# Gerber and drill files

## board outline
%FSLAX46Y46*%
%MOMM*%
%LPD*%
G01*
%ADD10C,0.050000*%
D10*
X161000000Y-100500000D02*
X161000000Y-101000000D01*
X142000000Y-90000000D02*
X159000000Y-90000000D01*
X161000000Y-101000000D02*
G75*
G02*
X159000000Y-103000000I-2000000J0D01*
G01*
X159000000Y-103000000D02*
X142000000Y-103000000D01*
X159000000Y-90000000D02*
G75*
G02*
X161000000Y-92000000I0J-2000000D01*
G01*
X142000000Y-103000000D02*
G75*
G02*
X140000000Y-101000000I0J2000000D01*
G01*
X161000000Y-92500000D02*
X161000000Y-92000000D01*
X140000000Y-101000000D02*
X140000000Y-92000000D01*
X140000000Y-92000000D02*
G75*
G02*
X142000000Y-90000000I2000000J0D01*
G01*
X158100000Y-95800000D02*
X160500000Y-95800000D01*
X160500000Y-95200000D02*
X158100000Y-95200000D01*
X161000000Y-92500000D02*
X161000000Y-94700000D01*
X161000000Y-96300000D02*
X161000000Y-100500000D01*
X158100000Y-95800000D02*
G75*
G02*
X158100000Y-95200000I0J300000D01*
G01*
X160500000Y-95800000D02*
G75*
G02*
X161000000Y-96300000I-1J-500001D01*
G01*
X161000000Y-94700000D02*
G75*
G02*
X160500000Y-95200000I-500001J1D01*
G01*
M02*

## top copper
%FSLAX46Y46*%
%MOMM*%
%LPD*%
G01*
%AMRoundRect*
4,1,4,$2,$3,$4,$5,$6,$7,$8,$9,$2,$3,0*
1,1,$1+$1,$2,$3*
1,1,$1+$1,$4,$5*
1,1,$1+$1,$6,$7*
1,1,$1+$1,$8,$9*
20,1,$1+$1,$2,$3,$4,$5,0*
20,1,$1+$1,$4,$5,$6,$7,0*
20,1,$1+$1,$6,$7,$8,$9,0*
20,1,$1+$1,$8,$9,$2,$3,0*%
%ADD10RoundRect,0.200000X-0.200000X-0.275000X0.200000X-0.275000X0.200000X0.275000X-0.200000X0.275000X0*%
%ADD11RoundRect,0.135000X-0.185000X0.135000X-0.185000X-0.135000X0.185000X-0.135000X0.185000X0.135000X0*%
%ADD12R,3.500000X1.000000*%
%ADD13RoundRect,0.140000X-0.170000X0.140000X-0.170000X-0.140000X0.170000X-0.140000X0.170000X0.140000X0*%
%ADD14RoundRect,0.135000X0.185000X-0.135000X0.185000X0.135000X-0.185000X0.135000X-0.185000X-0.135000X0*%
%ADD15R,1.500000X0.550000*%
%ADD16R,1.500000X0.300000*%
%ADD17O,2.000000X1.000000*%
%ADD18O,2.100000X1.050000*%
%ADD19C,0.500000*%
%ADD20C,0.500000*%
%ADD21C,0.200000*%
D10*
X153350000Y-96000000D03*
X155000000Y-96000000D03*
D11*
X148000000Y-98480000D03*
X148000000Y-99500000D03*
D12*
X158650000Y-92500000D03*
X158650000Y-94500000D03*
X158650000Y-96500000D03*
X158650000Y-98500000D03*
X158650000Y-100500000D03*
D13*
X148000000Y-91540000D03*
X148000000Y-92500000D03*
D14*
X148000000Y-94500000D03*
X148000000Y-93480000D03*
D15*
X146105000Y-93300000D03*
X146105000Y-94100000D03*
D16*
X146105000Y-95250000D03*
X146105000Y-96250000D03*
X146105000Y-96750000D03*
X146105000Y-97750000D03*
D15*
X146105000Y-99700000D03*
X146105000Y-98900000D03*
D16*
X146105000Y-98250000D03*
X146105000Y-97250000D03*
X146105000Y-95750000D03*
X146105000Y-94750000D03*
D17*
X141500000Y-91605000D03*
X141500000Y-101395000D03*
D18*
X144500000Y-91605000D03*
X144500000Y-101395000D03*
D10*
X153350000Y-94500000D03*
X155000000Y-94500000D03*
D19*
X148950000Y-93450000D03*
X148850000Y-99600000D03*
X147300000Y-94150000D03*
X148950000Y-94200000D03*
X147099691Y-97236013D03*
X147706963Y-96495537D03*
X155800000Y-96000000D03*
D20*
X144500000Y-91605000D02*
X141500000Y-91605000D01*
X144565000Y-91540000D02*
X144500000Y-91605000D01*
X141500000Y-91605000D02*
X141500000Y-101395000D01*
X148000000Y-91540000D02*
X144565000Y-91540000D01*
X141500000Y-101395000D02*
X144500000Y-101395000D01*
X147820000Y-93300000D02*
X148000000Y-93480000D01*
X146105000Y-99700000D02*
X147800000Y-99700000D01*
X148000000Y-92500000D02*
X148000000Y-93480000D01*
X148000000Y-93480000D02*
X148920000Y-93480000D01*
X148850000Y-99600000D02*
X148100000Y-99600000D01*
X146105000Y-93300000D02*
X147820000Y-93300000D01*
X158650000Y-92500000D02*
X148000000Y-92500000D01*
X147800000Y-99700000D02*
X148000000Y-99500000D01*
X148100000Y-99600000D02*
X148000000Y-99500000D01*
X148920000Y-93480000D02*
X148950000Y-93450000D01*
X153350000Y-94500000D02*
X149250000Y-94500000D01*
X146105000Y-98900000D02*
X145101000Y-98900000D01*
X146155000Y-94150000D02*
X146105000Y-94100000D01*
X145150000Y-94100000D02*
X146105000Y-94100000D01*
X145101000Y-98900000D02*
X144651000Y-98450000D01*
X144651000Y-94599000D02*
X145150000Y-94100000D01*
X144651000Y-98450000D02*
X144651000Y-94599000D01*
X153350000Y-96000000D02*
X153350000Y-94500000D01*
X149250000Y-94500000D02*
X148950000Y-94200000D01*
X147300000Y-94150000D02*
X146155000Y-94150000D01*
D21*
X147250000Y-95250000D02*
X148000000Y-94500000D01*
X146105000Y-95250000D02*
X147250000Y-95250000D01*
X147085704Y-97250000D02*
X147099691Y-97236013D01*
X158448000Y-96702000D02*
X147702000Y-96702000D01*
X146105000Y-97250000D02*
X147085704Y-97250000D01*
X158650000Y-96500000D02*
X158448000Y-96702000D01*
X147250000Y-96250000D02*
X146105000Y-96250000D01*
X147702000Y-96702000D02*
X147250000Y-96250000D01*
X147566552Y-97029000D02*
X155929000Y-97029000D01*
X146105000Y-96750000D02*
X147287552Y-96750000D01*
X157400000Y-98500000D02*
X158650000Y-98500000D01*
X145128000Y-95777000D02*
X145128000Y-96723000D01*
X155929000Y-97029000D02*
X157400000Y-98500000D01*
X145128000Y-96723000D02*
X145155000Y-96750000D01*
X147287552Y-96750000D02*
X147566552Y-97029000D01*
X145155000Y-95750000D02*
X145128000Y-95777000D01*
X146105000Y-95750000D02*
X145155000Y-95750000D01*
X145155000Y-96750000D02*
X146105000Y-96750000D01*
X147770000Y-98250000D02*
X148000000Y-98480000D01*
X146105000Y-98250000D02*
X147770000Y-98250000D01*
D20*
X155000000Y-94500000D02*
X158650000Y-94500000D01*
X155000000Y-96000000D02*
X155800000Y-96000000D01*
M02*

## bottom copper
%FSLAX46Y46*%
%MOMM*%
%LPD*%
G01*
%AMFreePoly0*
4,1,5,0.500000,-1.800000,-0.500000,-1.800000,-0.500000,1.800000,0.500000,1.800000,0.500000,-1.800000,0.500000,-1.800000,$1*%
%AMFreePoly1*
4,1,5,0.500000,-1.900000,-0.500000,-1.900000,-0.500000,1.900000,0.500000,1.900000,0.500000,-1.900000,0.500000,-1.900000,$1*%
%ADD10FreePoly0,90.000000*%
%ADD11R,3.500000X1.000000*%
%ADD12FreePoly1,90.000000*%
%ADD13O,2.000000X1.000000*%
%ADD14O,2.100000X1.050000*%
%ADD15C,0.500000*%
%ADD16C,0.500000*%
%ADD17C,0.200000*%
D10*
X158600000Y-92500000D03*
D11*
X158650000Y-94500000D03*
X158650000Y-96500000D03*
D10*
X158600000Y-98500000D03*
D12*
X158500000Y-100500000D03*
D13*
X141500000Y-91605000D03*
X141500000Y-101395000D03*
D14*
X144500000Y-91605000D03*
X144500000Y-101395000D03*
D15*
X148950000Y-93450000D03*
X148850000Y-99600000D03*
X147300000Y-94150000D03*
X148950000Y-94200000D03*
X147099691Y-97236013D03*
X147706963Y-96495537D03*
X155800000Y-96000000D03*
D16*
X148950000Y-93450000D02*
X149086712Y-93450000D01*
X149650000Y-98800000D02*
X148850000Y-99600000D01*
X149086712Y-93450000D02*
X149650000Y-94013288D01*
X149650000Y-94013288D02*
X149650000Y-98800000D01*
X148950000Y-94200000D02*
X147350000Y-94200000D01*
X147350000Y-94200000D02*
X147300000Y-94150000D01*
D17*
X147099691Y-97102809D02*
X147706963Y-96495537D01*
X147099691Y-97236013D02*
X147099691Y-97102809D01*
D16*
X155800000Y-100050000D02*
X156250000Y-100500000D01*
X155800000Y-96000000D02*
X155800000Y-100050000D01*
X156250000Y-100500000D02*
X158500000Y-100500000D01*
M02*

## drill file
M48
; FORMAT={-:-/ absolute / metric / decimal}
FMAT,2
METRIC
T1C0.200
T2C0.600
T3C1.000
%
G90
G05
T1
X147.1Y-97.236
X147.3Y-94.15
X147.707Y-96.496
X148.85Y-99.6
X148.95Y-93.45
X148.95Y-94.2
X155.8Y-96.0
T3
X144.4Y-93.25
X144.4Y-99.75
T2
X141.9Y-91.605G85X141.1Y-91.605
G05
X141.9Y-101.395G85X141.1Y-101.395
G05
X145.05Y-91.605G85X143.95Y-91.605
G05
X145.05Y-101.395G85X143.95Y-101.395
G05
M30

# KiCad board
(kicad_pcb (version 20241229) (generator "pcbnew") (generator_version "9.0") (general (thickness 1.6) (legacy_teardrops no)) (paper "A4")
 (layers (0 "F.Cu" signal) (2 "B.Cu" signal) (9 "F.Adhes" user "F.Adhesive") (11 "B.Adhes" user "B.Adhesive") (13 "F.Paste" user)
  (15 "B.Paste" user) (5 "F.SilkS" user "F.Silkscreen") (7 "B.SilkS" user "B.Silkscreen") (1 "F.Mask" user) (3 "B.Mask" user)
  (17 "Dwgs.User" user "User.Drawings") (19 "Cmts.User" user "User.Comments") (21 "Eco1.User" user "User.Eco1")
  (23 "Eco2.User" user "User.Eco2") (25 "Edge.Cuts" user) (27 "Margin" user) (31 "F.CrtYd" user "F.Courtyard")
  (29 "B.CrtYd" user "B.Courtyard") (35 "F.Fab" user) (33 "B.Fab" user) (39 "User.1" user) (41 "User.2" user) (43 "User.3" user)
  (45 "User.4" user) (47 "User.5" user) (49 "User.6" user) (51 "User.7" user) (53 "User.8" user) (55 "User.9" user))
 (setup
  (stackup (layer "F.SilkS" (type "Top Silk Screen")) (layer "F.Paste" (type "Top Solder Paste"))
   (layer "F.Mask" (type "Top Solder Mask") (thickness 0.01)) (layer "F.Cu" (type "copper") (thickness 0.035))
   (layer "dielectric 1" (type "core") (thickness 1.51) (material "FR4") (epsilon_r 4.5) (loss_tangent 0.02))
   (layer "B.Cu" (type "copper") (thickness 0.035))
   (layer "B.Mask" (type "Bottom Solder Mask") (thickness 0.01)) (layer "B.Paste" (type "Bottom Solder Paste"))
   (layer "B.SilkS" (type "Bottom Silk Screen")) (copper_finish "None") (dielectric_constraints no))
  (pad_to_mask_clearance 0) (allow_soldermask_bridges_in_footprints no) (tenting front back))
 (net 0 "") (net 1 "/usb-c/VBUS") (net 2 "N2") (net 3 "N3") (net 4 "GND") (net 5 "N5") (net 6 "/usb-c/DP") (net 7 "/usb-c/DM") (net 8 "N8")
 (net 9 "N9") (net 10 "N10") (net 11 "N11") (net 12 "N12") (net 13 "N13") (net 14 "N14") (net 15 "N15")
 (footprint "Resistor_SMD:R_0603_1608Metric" (layer "F.Cu") (at 154.175 96)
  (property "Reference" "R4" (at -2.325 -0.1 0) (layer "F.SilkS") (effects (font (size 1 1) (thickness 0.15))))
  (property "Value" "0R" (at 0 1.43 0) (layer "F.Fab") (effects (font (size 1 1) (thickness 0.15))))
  (pad "1" smd roundrect (at -0.825 0) (size 0.8 0.95) (layers "F.Cu" "F.Mask" "F.Paste") (roundrect_rratio 0.25) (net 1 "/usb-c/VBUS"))
  (pad "2" smd roundrect (at 0.825 0) (size 0.8 0.95) (layers "F.Cu" "F.Mask" "F.Paste") (roundrect_rratio 0.25) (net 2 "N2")))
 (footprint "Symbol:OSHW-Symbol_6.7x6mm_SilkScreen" (layer "F.Cu") (at 152 99.5)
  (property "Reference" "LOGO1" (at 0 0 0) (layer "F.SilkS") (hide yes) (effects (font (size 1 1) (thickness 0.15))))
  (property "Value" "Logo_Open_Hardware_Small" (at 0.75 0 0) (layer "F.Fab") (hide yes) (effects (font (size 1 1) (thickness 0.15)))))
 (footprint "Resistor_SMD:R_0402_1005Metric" (layer "F.Cu") (at 148 98.99 -90)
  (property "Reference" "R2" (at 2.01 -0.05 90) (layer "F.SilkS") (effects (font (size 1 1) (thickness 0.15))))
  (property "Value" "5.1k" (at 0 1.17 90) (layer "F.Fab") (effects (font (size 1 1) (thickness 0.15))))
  (pad "1" smd roundrect (at -0.51 0 270) (size 0.54 0.64) (layers "F.Cu" "F.Mask" "F.Paste") (roundrect_rratio 0.25) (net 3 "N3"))
  (pad "2" smd roundrect (at 0.51 0 270) (size 0.54 0.64) (layers "F.Cu" "F.Mask" "F.Paste") (roundrect_rratio 0.25) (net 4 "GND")))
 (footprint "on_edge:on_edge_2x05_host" (layer "F.Cu") (at 161 96.5 -90)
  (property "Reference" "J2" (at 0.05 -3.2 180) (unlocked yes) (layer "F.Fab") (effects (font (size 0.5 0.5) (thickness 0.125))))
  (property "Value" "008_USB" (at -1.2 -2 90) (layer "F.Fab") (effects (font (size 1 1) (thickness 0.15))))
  (fp_line (start -0.7 2.9) (end -0.7 0.5) (stroke (width 0.05) (type solid)) (layer "Edge.Cuts"))
  (fp_line (start -1.3 0.5) (end -1.3 2.9) (stroke (width 0.05) (type solid)) (layer "Edge.Cuts"))
  (fp_line (start -4 0) (end -1.8 0) (stroke (width 0.05) (type solid)) (layer "Edge.Cuts"))
  (fp_line (start -0.2 0) (end 4 0) (stroke (width 0.05) (type solid)) (layer "Edge.Cuts"))
  (fp_arc (start -0.7 2.9) (mid -1 3.2) (end -1.3 2.9) (stroke (width 0.05) (type solid)) (layer "Edge.Cuts"))
  (fp_arc (start -0.7 0.5) (mid -0.553553 0.146447) (end -0.2 0) (stroke (width 0.05) (type solid)) (layer "Edge.Cuts"))
  (fp_arc (start -1.8 0) (mid -1.446447 0.146447) (end -1.3 0.5) (stroke (width 0.05) (type solid)) (layer "Edge.Cuts"))
  (pad "1" smd rect (at -4 2.35 270) (size 1 3.5) (layers "F.Cu" "F.Mask") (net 4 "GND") (zone_connect 0))
  (pad "2" smd rect (at -2 2.35 270) (size 1 3.5) (layers "F.Cu" "F.Mask") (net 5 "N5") (zone_connect 0))
  (pad "3" smd rect (at 0 2.35 270) (size 1 3.5) (layers "F.Cu" "F.Mask") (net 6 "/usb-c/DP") (zone_connect 0))
  (pad "4" smd rect (at 2 2.35 270) (size 1 3.5) (layers "F.Cu" "F.Mask") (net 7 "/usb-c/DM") (zone_connect 0))
  (pad "5" smd rect (at 4 2.35 270) (size 1 3.5) (layers "F.Cu" "F.Mask") (zone_connect 0))
  (pad "6" smd custom (at -4 2.4 90) (size 1 3.6) (layers "B.Cu" "B.Mask") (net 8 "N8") (zone_connect 0)
   (options (clearance outline) (anchor rect)) (primitives))
  (pad "7" smd rect (at -2 2.35 90) (size 1 3.5) (layers "B.Cu" "B.Mask") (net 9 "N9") (zone_connect 0))
  (pad "8" smd rect (at 0 2.35 90) (size 1 3.5) (layers "B.Cu" "B.Mask") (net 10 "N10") (zone_connect 0))
  (pad "9" smd custom (at 2 2.4 90) (size 1 3.6) (layers "B.Cu" "B.Mask") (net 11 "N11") (zone_connect 0)
   (options (clearance outline) (anchor rect)) (primitives))
  (pad "10" smd custom (at 4 2.5 90) (size 1 3.8) (layers "B.Cu" "B.Mask") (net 2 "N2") (zone_connect 0)
   (options (clearance outline) (anchor rect)) (primitives))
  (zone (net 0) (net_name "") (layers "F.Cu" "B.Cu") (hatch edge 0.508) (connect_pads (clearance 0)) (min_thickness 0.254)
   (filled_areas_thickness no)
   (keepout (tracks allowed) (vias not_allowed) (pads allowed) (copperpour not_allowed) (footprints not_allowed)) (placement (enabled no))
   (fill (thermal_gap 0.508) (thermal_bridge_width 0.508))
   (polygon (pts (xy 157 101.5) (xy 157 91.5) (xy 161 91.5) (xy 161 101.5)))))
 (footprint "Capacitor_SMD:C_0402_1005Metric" (layer "F.Cu") (at 148 92.02 -90)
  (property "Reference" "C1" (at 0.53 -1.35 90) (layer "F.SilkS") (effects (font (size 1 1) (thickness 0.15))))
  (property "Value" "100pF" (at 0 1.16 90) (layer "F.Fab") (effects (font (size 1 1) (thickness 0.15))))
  (pad "1" smd roundrect (at -0.48 0 270) (size 0.56 0.62) (layers "F.Cu" "F.Mask" "F.Paste") (roundrect_rratio 0.25) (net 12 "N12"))
  (pad "2" smd roundrect (at 0.48 0 270) (size 0.56 0.62) (layers "F.Cu" "F.Mask" "F.Paste") (roundrect_rratio 0.25) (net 4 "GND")))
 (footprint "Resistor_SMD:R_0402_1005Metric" (layer "F.Cu") (at 148 93.99 90)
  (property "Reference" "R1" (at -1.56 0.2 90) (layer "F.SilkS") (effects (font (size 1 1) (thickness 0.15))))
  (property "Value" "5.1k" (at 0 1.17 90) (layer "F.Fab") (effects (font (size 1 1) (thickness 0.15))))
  (pad "1" smd roundrect (at -0.51 0 90) (size 0.54 0.64) (layers "F.Cu" "F.Mask" "F.Paste") (roundrect_rratio 0.25) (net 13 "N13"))
  (pad "2" smd roundrect (at 0.51 0 90) (size 0.54 0.64) (layers "F.Cu" "F.Mask" "F.Paste") (roundrect_rratio 0.25) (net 4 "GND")))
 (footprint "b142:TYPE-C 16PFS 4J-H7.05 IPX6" (layer "F.Cu") (at 143 96.5 -90)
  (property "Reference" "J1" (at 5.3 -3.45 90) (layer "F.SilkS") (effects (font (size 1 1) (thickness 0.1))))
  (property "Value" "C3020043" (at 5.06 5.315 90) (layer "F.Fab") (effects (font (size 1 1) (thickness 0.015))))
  (pad "" np_thru_hole circle (at -3.25 -1.4 270) (size 1 1) (drill 1) (layers "*.Cu" "*.Mask"))
  (pad "" np_thru_hole circle (at 3.25 -1.4 270) (size 1 1) (drill 1) (layers "*.Cu" "*.Mask"))
  (pad "A1/B12" smd rect (at -3.2 -3.105 270) (size 0.55 1.5) (layers "F.Cu" "F.Mask" "F.Paste") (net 4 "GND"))
  (pad "A4/B9" smd rect (at -2.4 -3.105 270) (size 0.55 1.5) (layers "F.Cu" "F.Mask" "F.Paste") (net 1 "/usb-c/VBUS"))
  (pad "A5" smd rect (at -1.25 -3.105 270) (size 0.3 1.5) (layers "F.Cu" "F.Mask" "F.Paste") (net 13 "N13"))
  (pad "A6" smd rect (at -0.25 -3.105 270) (size 0.3 1.5) (layers "F.Cu" "F.Mask" "F.Paste") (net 6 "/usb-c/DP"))
  (pad "A7" smd rect (at 0.25 -3.105 270) (size 0.3 1.5) (layers "F.Cu" "F.Mask" "F.Paste") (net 7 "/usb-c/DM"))
  (pad "A8" smd rect (at 1.25 -3.105 270) (size 0.3 1.5) (layers "F.Cu" "F.Mask" "F.Paste") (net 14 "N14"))
  (pad "B1/A12" smd rect (at 3.2 -3.105 270) (size 0.55 1.5) (layers "F.Cu" "F.Mask" "F.Paste") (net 4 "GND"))
  (pad "B4/A9" smd rect (at 2.4 -3.105 270) (size 0.55 1.5) (layers "F.Cu" "F.Mask" "F.Paste") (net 1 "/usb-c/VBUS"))
  (pad "B5" smd rect (at 1.75 -3.105 270) (size 0.3 1.5) (layers "F.Cu" "F.Mask" "F.Paste") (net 3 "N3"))
  (pad "B6" smd rect (at 0.75 -3.105 270) (size 0.3 1.5) (layers "F.Cu" "F.Mask" "F.Paste") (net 6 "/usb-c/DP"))
  (pad "B7" smd rect (at -0.75 -3.105 270) (size 0.3 1.5) (layers "F.Cu" "F.Mask" "F.Paste") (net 7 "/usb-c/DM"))
  (pad "B8" smd rect (at -1.75 -3.105 270) (size 0.3 1.5) (layers "F.Cu" "F.Mask" "F.Paste") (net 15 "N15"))
  (pad "G1" thru_hole oval (at -4.895 1.5 270) (size 1 2) (drill oval 0.6 1.4) (layers "*.Cu" "*.Mask") (remove_unused_layers no)
   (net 12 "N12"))
  (pad "G2" thru_hole oval (at 4.895 1.5 270) (size 1 2) (drill oval 0.6 1.4) (layers "*.Cu" "*.Mask") (remove_unused_layers no)
   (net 12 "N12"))
  (pad "G3" thru_hole oval (at -4.895 -1.5 270) (size 1.05 2.1) (drill oval 0.6 1.7) (layers "*.Cu" "*.Mask") (remove_unused_layers no)
   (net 12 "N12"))
  (pad "G4" thru_hole oval (at 4.895 -1.5 270) (size 1.05 2.1) (drill oval 0.6 1.7) (layers "*.Cu" "*.Mask") (remove_unused_layers no)
   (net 12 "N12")))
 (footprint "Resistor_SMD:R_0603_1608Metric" (layer "F.Cu") (at 154.175 94.5)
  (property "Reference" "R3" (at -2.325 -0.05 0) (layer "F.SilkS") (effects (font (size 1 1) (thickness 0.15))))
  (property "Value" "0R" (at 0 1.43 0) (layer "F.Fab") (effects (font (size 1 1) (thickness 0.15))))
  (pad "1" smd roundrect (at -0.825 0) (size 0.8 0.95) (layers "F.Cu" "F.Mask" "F.Paste") (roundrect_rratio 0.25) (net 1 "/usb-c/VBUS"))
  (pad "2" smd roundrect (at 0.825 0) (size 0.8 0.95) (layers "F.Cu" "F.Mask" "F.Paste") (roundrect_rratio 0.25) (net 5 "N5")))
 (gr_line (start 161 100.5) (end 161 101) (stroke (width 0.05) (type default)) (layer "Edge.Cuts"))
 (gr_line (start 142 90) (end 159 90) (stroke (width 0.05) (type solid)) (layer "Edge.Cuts"))
 (gr_arc (start 161 101) (mid 160.414214 102.414214) (end 159 103) (stroke (width 0.05) (type solid)) (layer "Edge.Cuts"))
 (gr_line (start 159 103) (end 142 103) (stroke (width 0.05) (type solid)) (layer "Edge.Cuts"))
 (gr_arc (start 159 90) (mid 160.414214 90.585786) (end 161 92) (stroke (width 0.05) (type solid)) (layer "Edge.Cuts"))
 (gr_arc (start 142 103) (mid 140.585786 102.414214) (end 140 101) (stroke (width 0.05) (type solid)) (layer "Edge.Cuts"))
 (gr_line (start 161 92.5) (end 161 92) (stroke (width 0.05) (type solid)) (layer "Edge.Cuts"))
 (gr_line (start 140 101) (end 140 92) (stroke (width 0.05) (type solid)) (layer "Edge.Cuts"))
 (gr_arc (start 140 92) (mid 140.585786 90.585786) (end 142 90) (stroke (width 0.05) (type solid)) (layer "Edge.Cuts"))
 (segment (start 144.5 91.605) (end 141.5 91.605) (width 0.5) (layer "F.Cu") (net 12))
 (segment (start 144.565 91.54) (end 144.5 91.605) (width 0.5) (layer "F.Cu") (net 12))
 (segment (start 141.5 91.605) (end 141.5 101.395) (width 0.5) (layer "F.Cu") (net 12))
 (segment (start 148 91.54) (end 144.565 91.54) (width 0.5) (layer "F.Cu") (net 12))
 (segment (start 141.5 101.395) (end 144.5 101.395) (width 0.5) (layer "F.Cu") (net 12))
 (segment (start 147.82 93.3) (end 148 93.48) (width 0.5) (layer "F.Cu") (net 4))
 (segment (start 146.105 99.7) (end 147.8 99.7) (width 0.5) (layer "F.Cu") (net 4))
 (segment (start 148 92.5) (end 148 93.48) (width 0.5) (layer "F.Cu") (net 4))
 (segment (start 148 93.48) (end 148.92 93.48) (width 0.5) (layer "F.Cu") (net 4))
 (segment (start 148.85 99.6) (end 148.1 99.6) (width 0.5) (layer "F.Cu") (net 4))
 (segment (start 146.105 93.3) (end 147.82 93.3) (width 0.5) (layer "F.Cu") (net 4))
 (segment (start 158.65 92.5) (end 148 92.5) (width 0.5) (layer "F.Cu") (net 4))
 (segment (start 147.8 99.7) (end 148 99.5) (width 0.5) (layer "F.Cu") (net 4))
 (segment (start 148.1 99.6) (end 148 99.5) (width 0.5) (layer "F.Cu") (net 4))
 (segment (start 148.92 93.48) (end 148.95 93.45) (width 0.5) (layer "F.Cu") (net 4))
 (via (at 148.95 93.45) (size 0.5) (drill 0.2) (layers "F.Cu" "B.Cu") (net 4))
 (via (at 148.85 99.6) (size 0.5) (drill 0.2) (layers "F.Cu" "B.Cu") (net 4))
 (segment (start 148.95 93.45) (end 149.086712 93.45) (width 0.5) (layer "B.Cu") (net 4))
 (segment (start 149.65 98.8) (end 148.85 99.6) (width 0.5) (layer "B.Cu") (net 4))
 (segment (start 149.086712 93.45) (end 149.65 94.013288) (width 0.5) (layer "B.Cu") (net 4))
 (segment (start 149.65 94.013288) (end 149.65 98.8) (width 0.5) (layer "B.Cu") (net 4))
 (segment (start 153.35 94.5) (end 149.25 94.5) (width 0.5) (layer "F.Cu") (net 1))
 (segment (start 146.105 98.9) (end 145.101 98.9) (width 0.5) (layer "F.Cu") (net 1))
 (segment (start 146.155 94.15) (end 146.105 94.1) (width 0.5) (layer "F.Cu") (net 1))
 (segment (start 145.15 94.1) (end 146.105 94.1) (width 0.5) (layer "F.Cu") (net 1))
 (segment (start 145.101 98.9) (end 144.651 98.45) (width 0.5) (layer "F.Cu") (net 1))
 (segment (start 144.651 94.599) (end 145.15 94.1) (width 0.5) (layer "F.Cu") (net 1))
 (segment (start 144.651 98.45) (end 144.651 94.599) (width 0.5) (layer "F.Cu") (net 1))
 (segment (start 153.35 96) (end 153.35 94.5) (width 0.5) (layer "F.Cu") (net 1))
 (segment (start 149.25 94.5) (end 148.95 94.2) (width 0.5) (layer "F.Cu") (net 1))
 (segment (start 147.3 94.15) (end 146.155 94.15) (width 0.5) (layer "F.Cu") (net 1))
 (via (at 147.3 94.15) (size 0.5) (drill 0.2) (layers "F.Cu" "B.Cu") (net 1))
 (via (at 148.95 94.2) (size 0.5) (drill 0.2) (layers "F.Cu" "B.Cu") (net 1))
 (segment (start 148.95 94.2) (end 147.35 94.2) (width 0.5) (layer "B.Cu") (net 1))
 (segment (start 147.35 94.2) (end 147.3 94.15) (width 0.5) (layer "B.Cu") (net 1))
 (segment (start 147.25 95.25) (end 148 94.5) (width 0.2) (layer "F.Cu") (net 13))
 (segment (start 146.105 95.25) (end 147.25 95.25) (width 0.2) (layer "F.Cu") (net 13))
 (segment (start 147.085704 97.25) (end 147.099691 97.236013) (width 0.2) (layer "F.Cu") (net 6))
 (segment (start 158.448 96.702) (end 147.702 96.702) (width 0.2) (layer "F.Cu") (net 6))
 (segment (start 146.105 97.25) (end 147.085704 97.25) (width 0.2) (layer "F.Cu") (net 6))
 (segment (start 158.65 96.5) (end 158.448 96.702) (width 0.2) (layer "F.Cu") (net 6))
 (segment (start 147.25 96.25) (end 146.105 96.25) (width 0.2) (layer "F.Cu") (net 6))
 (segment (start 147.702 96.702) (end 147.25 96.25) (width 0.2) (layer "F.Cu") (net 6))
 (via (at 147.099691 97.236013) (size 0.5) (drill 0.2) (layers "F.Cu" "B.Cu") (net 6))
 (via (at 147.706963 96.495537) (size 0.5) (drill 0.2) (layers "F.Cu" "B.Cu") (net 6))
 (segment (start 147.099691 97.102809) (end 147.706963 96.495537) (width 0.2) (layer "B.Cu") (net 6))
 (segment (start 147.099691 97.236013) (end 147.099691 97.102809) (width 0.2) (layer "B.Cu") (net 6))
 (segment (start 147.566552 97.029) (end 155.929 97.029) (width 0.2) (layer "F.Cu") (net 7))
 (segment (start 146.105 96.75) (end 147.287552 96.75) (width 0.2) (layer "F.Cu") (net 7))
 (segment (start 157.4 98.5) (end 158.65 98.5) (width 0.2) (layer "F.Cu") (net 7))
 (segment (start 145.128 95.777) (end 145.128 96.723) (width 0.2) (layer "F.Cu") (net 7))
 (segment (start 155.929 97.029) (end 157.4 98.5) (width 0.2) (layer "F.Cu") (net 7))
 (segment (start 145.128 96.723) (end 145.155 96.75) (width 0.2) (layer "F.Cu") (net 7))
 (segment (start 147.287552 96.75) (end 147.566552 97.029) (width 0.2) (layer "F.Cu") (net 7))
 (segment (start 145.155 95.75) (end 145.128 95.777) (width 0.2) (layer "F.Cu") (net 7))
 (segment (start 146.105 95.75) (end 145.155 95.75) (width 0.2) (layer "F.Cu") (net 7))
 (segment (start 145.155 96.75) (end 146.105 96.75) (width 0.2) (layer "F.Cu") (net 7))
 (segment (start 147.77 98.25) (end 148 98.48) (width 0.2) (layer "F.Cu") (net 3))
 (segment (start 146.105 98.25) (end 147.77 98.25) (width 0.2) (layer "F.Cu") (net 3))
 (segment (start 155 94.5) (end 158.65 94.5) (width 0.5) (layer "F.Cu") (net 5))
 (segment (start 155 96) (end 155.8 96) (width 0.5) (layer "F.Cu") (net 2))
 (via (at 155.8 96) (size 0.5) (drill 0.2) (layers "F.Cu" "B.Cu") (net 2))
 (segment (start 155.8 100.05) (end 156.25 100.5) (width 0.5) (layer "B.Cu") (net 2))
 (segment (start 155.8 96) (end 155.8 100.05) (width 0.5) (layer "B.Cu") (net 2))
 (segment (start 156.25 100.5) (end 158.5 100.5) (width 0.5) (layer "B.Cu") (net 2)))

